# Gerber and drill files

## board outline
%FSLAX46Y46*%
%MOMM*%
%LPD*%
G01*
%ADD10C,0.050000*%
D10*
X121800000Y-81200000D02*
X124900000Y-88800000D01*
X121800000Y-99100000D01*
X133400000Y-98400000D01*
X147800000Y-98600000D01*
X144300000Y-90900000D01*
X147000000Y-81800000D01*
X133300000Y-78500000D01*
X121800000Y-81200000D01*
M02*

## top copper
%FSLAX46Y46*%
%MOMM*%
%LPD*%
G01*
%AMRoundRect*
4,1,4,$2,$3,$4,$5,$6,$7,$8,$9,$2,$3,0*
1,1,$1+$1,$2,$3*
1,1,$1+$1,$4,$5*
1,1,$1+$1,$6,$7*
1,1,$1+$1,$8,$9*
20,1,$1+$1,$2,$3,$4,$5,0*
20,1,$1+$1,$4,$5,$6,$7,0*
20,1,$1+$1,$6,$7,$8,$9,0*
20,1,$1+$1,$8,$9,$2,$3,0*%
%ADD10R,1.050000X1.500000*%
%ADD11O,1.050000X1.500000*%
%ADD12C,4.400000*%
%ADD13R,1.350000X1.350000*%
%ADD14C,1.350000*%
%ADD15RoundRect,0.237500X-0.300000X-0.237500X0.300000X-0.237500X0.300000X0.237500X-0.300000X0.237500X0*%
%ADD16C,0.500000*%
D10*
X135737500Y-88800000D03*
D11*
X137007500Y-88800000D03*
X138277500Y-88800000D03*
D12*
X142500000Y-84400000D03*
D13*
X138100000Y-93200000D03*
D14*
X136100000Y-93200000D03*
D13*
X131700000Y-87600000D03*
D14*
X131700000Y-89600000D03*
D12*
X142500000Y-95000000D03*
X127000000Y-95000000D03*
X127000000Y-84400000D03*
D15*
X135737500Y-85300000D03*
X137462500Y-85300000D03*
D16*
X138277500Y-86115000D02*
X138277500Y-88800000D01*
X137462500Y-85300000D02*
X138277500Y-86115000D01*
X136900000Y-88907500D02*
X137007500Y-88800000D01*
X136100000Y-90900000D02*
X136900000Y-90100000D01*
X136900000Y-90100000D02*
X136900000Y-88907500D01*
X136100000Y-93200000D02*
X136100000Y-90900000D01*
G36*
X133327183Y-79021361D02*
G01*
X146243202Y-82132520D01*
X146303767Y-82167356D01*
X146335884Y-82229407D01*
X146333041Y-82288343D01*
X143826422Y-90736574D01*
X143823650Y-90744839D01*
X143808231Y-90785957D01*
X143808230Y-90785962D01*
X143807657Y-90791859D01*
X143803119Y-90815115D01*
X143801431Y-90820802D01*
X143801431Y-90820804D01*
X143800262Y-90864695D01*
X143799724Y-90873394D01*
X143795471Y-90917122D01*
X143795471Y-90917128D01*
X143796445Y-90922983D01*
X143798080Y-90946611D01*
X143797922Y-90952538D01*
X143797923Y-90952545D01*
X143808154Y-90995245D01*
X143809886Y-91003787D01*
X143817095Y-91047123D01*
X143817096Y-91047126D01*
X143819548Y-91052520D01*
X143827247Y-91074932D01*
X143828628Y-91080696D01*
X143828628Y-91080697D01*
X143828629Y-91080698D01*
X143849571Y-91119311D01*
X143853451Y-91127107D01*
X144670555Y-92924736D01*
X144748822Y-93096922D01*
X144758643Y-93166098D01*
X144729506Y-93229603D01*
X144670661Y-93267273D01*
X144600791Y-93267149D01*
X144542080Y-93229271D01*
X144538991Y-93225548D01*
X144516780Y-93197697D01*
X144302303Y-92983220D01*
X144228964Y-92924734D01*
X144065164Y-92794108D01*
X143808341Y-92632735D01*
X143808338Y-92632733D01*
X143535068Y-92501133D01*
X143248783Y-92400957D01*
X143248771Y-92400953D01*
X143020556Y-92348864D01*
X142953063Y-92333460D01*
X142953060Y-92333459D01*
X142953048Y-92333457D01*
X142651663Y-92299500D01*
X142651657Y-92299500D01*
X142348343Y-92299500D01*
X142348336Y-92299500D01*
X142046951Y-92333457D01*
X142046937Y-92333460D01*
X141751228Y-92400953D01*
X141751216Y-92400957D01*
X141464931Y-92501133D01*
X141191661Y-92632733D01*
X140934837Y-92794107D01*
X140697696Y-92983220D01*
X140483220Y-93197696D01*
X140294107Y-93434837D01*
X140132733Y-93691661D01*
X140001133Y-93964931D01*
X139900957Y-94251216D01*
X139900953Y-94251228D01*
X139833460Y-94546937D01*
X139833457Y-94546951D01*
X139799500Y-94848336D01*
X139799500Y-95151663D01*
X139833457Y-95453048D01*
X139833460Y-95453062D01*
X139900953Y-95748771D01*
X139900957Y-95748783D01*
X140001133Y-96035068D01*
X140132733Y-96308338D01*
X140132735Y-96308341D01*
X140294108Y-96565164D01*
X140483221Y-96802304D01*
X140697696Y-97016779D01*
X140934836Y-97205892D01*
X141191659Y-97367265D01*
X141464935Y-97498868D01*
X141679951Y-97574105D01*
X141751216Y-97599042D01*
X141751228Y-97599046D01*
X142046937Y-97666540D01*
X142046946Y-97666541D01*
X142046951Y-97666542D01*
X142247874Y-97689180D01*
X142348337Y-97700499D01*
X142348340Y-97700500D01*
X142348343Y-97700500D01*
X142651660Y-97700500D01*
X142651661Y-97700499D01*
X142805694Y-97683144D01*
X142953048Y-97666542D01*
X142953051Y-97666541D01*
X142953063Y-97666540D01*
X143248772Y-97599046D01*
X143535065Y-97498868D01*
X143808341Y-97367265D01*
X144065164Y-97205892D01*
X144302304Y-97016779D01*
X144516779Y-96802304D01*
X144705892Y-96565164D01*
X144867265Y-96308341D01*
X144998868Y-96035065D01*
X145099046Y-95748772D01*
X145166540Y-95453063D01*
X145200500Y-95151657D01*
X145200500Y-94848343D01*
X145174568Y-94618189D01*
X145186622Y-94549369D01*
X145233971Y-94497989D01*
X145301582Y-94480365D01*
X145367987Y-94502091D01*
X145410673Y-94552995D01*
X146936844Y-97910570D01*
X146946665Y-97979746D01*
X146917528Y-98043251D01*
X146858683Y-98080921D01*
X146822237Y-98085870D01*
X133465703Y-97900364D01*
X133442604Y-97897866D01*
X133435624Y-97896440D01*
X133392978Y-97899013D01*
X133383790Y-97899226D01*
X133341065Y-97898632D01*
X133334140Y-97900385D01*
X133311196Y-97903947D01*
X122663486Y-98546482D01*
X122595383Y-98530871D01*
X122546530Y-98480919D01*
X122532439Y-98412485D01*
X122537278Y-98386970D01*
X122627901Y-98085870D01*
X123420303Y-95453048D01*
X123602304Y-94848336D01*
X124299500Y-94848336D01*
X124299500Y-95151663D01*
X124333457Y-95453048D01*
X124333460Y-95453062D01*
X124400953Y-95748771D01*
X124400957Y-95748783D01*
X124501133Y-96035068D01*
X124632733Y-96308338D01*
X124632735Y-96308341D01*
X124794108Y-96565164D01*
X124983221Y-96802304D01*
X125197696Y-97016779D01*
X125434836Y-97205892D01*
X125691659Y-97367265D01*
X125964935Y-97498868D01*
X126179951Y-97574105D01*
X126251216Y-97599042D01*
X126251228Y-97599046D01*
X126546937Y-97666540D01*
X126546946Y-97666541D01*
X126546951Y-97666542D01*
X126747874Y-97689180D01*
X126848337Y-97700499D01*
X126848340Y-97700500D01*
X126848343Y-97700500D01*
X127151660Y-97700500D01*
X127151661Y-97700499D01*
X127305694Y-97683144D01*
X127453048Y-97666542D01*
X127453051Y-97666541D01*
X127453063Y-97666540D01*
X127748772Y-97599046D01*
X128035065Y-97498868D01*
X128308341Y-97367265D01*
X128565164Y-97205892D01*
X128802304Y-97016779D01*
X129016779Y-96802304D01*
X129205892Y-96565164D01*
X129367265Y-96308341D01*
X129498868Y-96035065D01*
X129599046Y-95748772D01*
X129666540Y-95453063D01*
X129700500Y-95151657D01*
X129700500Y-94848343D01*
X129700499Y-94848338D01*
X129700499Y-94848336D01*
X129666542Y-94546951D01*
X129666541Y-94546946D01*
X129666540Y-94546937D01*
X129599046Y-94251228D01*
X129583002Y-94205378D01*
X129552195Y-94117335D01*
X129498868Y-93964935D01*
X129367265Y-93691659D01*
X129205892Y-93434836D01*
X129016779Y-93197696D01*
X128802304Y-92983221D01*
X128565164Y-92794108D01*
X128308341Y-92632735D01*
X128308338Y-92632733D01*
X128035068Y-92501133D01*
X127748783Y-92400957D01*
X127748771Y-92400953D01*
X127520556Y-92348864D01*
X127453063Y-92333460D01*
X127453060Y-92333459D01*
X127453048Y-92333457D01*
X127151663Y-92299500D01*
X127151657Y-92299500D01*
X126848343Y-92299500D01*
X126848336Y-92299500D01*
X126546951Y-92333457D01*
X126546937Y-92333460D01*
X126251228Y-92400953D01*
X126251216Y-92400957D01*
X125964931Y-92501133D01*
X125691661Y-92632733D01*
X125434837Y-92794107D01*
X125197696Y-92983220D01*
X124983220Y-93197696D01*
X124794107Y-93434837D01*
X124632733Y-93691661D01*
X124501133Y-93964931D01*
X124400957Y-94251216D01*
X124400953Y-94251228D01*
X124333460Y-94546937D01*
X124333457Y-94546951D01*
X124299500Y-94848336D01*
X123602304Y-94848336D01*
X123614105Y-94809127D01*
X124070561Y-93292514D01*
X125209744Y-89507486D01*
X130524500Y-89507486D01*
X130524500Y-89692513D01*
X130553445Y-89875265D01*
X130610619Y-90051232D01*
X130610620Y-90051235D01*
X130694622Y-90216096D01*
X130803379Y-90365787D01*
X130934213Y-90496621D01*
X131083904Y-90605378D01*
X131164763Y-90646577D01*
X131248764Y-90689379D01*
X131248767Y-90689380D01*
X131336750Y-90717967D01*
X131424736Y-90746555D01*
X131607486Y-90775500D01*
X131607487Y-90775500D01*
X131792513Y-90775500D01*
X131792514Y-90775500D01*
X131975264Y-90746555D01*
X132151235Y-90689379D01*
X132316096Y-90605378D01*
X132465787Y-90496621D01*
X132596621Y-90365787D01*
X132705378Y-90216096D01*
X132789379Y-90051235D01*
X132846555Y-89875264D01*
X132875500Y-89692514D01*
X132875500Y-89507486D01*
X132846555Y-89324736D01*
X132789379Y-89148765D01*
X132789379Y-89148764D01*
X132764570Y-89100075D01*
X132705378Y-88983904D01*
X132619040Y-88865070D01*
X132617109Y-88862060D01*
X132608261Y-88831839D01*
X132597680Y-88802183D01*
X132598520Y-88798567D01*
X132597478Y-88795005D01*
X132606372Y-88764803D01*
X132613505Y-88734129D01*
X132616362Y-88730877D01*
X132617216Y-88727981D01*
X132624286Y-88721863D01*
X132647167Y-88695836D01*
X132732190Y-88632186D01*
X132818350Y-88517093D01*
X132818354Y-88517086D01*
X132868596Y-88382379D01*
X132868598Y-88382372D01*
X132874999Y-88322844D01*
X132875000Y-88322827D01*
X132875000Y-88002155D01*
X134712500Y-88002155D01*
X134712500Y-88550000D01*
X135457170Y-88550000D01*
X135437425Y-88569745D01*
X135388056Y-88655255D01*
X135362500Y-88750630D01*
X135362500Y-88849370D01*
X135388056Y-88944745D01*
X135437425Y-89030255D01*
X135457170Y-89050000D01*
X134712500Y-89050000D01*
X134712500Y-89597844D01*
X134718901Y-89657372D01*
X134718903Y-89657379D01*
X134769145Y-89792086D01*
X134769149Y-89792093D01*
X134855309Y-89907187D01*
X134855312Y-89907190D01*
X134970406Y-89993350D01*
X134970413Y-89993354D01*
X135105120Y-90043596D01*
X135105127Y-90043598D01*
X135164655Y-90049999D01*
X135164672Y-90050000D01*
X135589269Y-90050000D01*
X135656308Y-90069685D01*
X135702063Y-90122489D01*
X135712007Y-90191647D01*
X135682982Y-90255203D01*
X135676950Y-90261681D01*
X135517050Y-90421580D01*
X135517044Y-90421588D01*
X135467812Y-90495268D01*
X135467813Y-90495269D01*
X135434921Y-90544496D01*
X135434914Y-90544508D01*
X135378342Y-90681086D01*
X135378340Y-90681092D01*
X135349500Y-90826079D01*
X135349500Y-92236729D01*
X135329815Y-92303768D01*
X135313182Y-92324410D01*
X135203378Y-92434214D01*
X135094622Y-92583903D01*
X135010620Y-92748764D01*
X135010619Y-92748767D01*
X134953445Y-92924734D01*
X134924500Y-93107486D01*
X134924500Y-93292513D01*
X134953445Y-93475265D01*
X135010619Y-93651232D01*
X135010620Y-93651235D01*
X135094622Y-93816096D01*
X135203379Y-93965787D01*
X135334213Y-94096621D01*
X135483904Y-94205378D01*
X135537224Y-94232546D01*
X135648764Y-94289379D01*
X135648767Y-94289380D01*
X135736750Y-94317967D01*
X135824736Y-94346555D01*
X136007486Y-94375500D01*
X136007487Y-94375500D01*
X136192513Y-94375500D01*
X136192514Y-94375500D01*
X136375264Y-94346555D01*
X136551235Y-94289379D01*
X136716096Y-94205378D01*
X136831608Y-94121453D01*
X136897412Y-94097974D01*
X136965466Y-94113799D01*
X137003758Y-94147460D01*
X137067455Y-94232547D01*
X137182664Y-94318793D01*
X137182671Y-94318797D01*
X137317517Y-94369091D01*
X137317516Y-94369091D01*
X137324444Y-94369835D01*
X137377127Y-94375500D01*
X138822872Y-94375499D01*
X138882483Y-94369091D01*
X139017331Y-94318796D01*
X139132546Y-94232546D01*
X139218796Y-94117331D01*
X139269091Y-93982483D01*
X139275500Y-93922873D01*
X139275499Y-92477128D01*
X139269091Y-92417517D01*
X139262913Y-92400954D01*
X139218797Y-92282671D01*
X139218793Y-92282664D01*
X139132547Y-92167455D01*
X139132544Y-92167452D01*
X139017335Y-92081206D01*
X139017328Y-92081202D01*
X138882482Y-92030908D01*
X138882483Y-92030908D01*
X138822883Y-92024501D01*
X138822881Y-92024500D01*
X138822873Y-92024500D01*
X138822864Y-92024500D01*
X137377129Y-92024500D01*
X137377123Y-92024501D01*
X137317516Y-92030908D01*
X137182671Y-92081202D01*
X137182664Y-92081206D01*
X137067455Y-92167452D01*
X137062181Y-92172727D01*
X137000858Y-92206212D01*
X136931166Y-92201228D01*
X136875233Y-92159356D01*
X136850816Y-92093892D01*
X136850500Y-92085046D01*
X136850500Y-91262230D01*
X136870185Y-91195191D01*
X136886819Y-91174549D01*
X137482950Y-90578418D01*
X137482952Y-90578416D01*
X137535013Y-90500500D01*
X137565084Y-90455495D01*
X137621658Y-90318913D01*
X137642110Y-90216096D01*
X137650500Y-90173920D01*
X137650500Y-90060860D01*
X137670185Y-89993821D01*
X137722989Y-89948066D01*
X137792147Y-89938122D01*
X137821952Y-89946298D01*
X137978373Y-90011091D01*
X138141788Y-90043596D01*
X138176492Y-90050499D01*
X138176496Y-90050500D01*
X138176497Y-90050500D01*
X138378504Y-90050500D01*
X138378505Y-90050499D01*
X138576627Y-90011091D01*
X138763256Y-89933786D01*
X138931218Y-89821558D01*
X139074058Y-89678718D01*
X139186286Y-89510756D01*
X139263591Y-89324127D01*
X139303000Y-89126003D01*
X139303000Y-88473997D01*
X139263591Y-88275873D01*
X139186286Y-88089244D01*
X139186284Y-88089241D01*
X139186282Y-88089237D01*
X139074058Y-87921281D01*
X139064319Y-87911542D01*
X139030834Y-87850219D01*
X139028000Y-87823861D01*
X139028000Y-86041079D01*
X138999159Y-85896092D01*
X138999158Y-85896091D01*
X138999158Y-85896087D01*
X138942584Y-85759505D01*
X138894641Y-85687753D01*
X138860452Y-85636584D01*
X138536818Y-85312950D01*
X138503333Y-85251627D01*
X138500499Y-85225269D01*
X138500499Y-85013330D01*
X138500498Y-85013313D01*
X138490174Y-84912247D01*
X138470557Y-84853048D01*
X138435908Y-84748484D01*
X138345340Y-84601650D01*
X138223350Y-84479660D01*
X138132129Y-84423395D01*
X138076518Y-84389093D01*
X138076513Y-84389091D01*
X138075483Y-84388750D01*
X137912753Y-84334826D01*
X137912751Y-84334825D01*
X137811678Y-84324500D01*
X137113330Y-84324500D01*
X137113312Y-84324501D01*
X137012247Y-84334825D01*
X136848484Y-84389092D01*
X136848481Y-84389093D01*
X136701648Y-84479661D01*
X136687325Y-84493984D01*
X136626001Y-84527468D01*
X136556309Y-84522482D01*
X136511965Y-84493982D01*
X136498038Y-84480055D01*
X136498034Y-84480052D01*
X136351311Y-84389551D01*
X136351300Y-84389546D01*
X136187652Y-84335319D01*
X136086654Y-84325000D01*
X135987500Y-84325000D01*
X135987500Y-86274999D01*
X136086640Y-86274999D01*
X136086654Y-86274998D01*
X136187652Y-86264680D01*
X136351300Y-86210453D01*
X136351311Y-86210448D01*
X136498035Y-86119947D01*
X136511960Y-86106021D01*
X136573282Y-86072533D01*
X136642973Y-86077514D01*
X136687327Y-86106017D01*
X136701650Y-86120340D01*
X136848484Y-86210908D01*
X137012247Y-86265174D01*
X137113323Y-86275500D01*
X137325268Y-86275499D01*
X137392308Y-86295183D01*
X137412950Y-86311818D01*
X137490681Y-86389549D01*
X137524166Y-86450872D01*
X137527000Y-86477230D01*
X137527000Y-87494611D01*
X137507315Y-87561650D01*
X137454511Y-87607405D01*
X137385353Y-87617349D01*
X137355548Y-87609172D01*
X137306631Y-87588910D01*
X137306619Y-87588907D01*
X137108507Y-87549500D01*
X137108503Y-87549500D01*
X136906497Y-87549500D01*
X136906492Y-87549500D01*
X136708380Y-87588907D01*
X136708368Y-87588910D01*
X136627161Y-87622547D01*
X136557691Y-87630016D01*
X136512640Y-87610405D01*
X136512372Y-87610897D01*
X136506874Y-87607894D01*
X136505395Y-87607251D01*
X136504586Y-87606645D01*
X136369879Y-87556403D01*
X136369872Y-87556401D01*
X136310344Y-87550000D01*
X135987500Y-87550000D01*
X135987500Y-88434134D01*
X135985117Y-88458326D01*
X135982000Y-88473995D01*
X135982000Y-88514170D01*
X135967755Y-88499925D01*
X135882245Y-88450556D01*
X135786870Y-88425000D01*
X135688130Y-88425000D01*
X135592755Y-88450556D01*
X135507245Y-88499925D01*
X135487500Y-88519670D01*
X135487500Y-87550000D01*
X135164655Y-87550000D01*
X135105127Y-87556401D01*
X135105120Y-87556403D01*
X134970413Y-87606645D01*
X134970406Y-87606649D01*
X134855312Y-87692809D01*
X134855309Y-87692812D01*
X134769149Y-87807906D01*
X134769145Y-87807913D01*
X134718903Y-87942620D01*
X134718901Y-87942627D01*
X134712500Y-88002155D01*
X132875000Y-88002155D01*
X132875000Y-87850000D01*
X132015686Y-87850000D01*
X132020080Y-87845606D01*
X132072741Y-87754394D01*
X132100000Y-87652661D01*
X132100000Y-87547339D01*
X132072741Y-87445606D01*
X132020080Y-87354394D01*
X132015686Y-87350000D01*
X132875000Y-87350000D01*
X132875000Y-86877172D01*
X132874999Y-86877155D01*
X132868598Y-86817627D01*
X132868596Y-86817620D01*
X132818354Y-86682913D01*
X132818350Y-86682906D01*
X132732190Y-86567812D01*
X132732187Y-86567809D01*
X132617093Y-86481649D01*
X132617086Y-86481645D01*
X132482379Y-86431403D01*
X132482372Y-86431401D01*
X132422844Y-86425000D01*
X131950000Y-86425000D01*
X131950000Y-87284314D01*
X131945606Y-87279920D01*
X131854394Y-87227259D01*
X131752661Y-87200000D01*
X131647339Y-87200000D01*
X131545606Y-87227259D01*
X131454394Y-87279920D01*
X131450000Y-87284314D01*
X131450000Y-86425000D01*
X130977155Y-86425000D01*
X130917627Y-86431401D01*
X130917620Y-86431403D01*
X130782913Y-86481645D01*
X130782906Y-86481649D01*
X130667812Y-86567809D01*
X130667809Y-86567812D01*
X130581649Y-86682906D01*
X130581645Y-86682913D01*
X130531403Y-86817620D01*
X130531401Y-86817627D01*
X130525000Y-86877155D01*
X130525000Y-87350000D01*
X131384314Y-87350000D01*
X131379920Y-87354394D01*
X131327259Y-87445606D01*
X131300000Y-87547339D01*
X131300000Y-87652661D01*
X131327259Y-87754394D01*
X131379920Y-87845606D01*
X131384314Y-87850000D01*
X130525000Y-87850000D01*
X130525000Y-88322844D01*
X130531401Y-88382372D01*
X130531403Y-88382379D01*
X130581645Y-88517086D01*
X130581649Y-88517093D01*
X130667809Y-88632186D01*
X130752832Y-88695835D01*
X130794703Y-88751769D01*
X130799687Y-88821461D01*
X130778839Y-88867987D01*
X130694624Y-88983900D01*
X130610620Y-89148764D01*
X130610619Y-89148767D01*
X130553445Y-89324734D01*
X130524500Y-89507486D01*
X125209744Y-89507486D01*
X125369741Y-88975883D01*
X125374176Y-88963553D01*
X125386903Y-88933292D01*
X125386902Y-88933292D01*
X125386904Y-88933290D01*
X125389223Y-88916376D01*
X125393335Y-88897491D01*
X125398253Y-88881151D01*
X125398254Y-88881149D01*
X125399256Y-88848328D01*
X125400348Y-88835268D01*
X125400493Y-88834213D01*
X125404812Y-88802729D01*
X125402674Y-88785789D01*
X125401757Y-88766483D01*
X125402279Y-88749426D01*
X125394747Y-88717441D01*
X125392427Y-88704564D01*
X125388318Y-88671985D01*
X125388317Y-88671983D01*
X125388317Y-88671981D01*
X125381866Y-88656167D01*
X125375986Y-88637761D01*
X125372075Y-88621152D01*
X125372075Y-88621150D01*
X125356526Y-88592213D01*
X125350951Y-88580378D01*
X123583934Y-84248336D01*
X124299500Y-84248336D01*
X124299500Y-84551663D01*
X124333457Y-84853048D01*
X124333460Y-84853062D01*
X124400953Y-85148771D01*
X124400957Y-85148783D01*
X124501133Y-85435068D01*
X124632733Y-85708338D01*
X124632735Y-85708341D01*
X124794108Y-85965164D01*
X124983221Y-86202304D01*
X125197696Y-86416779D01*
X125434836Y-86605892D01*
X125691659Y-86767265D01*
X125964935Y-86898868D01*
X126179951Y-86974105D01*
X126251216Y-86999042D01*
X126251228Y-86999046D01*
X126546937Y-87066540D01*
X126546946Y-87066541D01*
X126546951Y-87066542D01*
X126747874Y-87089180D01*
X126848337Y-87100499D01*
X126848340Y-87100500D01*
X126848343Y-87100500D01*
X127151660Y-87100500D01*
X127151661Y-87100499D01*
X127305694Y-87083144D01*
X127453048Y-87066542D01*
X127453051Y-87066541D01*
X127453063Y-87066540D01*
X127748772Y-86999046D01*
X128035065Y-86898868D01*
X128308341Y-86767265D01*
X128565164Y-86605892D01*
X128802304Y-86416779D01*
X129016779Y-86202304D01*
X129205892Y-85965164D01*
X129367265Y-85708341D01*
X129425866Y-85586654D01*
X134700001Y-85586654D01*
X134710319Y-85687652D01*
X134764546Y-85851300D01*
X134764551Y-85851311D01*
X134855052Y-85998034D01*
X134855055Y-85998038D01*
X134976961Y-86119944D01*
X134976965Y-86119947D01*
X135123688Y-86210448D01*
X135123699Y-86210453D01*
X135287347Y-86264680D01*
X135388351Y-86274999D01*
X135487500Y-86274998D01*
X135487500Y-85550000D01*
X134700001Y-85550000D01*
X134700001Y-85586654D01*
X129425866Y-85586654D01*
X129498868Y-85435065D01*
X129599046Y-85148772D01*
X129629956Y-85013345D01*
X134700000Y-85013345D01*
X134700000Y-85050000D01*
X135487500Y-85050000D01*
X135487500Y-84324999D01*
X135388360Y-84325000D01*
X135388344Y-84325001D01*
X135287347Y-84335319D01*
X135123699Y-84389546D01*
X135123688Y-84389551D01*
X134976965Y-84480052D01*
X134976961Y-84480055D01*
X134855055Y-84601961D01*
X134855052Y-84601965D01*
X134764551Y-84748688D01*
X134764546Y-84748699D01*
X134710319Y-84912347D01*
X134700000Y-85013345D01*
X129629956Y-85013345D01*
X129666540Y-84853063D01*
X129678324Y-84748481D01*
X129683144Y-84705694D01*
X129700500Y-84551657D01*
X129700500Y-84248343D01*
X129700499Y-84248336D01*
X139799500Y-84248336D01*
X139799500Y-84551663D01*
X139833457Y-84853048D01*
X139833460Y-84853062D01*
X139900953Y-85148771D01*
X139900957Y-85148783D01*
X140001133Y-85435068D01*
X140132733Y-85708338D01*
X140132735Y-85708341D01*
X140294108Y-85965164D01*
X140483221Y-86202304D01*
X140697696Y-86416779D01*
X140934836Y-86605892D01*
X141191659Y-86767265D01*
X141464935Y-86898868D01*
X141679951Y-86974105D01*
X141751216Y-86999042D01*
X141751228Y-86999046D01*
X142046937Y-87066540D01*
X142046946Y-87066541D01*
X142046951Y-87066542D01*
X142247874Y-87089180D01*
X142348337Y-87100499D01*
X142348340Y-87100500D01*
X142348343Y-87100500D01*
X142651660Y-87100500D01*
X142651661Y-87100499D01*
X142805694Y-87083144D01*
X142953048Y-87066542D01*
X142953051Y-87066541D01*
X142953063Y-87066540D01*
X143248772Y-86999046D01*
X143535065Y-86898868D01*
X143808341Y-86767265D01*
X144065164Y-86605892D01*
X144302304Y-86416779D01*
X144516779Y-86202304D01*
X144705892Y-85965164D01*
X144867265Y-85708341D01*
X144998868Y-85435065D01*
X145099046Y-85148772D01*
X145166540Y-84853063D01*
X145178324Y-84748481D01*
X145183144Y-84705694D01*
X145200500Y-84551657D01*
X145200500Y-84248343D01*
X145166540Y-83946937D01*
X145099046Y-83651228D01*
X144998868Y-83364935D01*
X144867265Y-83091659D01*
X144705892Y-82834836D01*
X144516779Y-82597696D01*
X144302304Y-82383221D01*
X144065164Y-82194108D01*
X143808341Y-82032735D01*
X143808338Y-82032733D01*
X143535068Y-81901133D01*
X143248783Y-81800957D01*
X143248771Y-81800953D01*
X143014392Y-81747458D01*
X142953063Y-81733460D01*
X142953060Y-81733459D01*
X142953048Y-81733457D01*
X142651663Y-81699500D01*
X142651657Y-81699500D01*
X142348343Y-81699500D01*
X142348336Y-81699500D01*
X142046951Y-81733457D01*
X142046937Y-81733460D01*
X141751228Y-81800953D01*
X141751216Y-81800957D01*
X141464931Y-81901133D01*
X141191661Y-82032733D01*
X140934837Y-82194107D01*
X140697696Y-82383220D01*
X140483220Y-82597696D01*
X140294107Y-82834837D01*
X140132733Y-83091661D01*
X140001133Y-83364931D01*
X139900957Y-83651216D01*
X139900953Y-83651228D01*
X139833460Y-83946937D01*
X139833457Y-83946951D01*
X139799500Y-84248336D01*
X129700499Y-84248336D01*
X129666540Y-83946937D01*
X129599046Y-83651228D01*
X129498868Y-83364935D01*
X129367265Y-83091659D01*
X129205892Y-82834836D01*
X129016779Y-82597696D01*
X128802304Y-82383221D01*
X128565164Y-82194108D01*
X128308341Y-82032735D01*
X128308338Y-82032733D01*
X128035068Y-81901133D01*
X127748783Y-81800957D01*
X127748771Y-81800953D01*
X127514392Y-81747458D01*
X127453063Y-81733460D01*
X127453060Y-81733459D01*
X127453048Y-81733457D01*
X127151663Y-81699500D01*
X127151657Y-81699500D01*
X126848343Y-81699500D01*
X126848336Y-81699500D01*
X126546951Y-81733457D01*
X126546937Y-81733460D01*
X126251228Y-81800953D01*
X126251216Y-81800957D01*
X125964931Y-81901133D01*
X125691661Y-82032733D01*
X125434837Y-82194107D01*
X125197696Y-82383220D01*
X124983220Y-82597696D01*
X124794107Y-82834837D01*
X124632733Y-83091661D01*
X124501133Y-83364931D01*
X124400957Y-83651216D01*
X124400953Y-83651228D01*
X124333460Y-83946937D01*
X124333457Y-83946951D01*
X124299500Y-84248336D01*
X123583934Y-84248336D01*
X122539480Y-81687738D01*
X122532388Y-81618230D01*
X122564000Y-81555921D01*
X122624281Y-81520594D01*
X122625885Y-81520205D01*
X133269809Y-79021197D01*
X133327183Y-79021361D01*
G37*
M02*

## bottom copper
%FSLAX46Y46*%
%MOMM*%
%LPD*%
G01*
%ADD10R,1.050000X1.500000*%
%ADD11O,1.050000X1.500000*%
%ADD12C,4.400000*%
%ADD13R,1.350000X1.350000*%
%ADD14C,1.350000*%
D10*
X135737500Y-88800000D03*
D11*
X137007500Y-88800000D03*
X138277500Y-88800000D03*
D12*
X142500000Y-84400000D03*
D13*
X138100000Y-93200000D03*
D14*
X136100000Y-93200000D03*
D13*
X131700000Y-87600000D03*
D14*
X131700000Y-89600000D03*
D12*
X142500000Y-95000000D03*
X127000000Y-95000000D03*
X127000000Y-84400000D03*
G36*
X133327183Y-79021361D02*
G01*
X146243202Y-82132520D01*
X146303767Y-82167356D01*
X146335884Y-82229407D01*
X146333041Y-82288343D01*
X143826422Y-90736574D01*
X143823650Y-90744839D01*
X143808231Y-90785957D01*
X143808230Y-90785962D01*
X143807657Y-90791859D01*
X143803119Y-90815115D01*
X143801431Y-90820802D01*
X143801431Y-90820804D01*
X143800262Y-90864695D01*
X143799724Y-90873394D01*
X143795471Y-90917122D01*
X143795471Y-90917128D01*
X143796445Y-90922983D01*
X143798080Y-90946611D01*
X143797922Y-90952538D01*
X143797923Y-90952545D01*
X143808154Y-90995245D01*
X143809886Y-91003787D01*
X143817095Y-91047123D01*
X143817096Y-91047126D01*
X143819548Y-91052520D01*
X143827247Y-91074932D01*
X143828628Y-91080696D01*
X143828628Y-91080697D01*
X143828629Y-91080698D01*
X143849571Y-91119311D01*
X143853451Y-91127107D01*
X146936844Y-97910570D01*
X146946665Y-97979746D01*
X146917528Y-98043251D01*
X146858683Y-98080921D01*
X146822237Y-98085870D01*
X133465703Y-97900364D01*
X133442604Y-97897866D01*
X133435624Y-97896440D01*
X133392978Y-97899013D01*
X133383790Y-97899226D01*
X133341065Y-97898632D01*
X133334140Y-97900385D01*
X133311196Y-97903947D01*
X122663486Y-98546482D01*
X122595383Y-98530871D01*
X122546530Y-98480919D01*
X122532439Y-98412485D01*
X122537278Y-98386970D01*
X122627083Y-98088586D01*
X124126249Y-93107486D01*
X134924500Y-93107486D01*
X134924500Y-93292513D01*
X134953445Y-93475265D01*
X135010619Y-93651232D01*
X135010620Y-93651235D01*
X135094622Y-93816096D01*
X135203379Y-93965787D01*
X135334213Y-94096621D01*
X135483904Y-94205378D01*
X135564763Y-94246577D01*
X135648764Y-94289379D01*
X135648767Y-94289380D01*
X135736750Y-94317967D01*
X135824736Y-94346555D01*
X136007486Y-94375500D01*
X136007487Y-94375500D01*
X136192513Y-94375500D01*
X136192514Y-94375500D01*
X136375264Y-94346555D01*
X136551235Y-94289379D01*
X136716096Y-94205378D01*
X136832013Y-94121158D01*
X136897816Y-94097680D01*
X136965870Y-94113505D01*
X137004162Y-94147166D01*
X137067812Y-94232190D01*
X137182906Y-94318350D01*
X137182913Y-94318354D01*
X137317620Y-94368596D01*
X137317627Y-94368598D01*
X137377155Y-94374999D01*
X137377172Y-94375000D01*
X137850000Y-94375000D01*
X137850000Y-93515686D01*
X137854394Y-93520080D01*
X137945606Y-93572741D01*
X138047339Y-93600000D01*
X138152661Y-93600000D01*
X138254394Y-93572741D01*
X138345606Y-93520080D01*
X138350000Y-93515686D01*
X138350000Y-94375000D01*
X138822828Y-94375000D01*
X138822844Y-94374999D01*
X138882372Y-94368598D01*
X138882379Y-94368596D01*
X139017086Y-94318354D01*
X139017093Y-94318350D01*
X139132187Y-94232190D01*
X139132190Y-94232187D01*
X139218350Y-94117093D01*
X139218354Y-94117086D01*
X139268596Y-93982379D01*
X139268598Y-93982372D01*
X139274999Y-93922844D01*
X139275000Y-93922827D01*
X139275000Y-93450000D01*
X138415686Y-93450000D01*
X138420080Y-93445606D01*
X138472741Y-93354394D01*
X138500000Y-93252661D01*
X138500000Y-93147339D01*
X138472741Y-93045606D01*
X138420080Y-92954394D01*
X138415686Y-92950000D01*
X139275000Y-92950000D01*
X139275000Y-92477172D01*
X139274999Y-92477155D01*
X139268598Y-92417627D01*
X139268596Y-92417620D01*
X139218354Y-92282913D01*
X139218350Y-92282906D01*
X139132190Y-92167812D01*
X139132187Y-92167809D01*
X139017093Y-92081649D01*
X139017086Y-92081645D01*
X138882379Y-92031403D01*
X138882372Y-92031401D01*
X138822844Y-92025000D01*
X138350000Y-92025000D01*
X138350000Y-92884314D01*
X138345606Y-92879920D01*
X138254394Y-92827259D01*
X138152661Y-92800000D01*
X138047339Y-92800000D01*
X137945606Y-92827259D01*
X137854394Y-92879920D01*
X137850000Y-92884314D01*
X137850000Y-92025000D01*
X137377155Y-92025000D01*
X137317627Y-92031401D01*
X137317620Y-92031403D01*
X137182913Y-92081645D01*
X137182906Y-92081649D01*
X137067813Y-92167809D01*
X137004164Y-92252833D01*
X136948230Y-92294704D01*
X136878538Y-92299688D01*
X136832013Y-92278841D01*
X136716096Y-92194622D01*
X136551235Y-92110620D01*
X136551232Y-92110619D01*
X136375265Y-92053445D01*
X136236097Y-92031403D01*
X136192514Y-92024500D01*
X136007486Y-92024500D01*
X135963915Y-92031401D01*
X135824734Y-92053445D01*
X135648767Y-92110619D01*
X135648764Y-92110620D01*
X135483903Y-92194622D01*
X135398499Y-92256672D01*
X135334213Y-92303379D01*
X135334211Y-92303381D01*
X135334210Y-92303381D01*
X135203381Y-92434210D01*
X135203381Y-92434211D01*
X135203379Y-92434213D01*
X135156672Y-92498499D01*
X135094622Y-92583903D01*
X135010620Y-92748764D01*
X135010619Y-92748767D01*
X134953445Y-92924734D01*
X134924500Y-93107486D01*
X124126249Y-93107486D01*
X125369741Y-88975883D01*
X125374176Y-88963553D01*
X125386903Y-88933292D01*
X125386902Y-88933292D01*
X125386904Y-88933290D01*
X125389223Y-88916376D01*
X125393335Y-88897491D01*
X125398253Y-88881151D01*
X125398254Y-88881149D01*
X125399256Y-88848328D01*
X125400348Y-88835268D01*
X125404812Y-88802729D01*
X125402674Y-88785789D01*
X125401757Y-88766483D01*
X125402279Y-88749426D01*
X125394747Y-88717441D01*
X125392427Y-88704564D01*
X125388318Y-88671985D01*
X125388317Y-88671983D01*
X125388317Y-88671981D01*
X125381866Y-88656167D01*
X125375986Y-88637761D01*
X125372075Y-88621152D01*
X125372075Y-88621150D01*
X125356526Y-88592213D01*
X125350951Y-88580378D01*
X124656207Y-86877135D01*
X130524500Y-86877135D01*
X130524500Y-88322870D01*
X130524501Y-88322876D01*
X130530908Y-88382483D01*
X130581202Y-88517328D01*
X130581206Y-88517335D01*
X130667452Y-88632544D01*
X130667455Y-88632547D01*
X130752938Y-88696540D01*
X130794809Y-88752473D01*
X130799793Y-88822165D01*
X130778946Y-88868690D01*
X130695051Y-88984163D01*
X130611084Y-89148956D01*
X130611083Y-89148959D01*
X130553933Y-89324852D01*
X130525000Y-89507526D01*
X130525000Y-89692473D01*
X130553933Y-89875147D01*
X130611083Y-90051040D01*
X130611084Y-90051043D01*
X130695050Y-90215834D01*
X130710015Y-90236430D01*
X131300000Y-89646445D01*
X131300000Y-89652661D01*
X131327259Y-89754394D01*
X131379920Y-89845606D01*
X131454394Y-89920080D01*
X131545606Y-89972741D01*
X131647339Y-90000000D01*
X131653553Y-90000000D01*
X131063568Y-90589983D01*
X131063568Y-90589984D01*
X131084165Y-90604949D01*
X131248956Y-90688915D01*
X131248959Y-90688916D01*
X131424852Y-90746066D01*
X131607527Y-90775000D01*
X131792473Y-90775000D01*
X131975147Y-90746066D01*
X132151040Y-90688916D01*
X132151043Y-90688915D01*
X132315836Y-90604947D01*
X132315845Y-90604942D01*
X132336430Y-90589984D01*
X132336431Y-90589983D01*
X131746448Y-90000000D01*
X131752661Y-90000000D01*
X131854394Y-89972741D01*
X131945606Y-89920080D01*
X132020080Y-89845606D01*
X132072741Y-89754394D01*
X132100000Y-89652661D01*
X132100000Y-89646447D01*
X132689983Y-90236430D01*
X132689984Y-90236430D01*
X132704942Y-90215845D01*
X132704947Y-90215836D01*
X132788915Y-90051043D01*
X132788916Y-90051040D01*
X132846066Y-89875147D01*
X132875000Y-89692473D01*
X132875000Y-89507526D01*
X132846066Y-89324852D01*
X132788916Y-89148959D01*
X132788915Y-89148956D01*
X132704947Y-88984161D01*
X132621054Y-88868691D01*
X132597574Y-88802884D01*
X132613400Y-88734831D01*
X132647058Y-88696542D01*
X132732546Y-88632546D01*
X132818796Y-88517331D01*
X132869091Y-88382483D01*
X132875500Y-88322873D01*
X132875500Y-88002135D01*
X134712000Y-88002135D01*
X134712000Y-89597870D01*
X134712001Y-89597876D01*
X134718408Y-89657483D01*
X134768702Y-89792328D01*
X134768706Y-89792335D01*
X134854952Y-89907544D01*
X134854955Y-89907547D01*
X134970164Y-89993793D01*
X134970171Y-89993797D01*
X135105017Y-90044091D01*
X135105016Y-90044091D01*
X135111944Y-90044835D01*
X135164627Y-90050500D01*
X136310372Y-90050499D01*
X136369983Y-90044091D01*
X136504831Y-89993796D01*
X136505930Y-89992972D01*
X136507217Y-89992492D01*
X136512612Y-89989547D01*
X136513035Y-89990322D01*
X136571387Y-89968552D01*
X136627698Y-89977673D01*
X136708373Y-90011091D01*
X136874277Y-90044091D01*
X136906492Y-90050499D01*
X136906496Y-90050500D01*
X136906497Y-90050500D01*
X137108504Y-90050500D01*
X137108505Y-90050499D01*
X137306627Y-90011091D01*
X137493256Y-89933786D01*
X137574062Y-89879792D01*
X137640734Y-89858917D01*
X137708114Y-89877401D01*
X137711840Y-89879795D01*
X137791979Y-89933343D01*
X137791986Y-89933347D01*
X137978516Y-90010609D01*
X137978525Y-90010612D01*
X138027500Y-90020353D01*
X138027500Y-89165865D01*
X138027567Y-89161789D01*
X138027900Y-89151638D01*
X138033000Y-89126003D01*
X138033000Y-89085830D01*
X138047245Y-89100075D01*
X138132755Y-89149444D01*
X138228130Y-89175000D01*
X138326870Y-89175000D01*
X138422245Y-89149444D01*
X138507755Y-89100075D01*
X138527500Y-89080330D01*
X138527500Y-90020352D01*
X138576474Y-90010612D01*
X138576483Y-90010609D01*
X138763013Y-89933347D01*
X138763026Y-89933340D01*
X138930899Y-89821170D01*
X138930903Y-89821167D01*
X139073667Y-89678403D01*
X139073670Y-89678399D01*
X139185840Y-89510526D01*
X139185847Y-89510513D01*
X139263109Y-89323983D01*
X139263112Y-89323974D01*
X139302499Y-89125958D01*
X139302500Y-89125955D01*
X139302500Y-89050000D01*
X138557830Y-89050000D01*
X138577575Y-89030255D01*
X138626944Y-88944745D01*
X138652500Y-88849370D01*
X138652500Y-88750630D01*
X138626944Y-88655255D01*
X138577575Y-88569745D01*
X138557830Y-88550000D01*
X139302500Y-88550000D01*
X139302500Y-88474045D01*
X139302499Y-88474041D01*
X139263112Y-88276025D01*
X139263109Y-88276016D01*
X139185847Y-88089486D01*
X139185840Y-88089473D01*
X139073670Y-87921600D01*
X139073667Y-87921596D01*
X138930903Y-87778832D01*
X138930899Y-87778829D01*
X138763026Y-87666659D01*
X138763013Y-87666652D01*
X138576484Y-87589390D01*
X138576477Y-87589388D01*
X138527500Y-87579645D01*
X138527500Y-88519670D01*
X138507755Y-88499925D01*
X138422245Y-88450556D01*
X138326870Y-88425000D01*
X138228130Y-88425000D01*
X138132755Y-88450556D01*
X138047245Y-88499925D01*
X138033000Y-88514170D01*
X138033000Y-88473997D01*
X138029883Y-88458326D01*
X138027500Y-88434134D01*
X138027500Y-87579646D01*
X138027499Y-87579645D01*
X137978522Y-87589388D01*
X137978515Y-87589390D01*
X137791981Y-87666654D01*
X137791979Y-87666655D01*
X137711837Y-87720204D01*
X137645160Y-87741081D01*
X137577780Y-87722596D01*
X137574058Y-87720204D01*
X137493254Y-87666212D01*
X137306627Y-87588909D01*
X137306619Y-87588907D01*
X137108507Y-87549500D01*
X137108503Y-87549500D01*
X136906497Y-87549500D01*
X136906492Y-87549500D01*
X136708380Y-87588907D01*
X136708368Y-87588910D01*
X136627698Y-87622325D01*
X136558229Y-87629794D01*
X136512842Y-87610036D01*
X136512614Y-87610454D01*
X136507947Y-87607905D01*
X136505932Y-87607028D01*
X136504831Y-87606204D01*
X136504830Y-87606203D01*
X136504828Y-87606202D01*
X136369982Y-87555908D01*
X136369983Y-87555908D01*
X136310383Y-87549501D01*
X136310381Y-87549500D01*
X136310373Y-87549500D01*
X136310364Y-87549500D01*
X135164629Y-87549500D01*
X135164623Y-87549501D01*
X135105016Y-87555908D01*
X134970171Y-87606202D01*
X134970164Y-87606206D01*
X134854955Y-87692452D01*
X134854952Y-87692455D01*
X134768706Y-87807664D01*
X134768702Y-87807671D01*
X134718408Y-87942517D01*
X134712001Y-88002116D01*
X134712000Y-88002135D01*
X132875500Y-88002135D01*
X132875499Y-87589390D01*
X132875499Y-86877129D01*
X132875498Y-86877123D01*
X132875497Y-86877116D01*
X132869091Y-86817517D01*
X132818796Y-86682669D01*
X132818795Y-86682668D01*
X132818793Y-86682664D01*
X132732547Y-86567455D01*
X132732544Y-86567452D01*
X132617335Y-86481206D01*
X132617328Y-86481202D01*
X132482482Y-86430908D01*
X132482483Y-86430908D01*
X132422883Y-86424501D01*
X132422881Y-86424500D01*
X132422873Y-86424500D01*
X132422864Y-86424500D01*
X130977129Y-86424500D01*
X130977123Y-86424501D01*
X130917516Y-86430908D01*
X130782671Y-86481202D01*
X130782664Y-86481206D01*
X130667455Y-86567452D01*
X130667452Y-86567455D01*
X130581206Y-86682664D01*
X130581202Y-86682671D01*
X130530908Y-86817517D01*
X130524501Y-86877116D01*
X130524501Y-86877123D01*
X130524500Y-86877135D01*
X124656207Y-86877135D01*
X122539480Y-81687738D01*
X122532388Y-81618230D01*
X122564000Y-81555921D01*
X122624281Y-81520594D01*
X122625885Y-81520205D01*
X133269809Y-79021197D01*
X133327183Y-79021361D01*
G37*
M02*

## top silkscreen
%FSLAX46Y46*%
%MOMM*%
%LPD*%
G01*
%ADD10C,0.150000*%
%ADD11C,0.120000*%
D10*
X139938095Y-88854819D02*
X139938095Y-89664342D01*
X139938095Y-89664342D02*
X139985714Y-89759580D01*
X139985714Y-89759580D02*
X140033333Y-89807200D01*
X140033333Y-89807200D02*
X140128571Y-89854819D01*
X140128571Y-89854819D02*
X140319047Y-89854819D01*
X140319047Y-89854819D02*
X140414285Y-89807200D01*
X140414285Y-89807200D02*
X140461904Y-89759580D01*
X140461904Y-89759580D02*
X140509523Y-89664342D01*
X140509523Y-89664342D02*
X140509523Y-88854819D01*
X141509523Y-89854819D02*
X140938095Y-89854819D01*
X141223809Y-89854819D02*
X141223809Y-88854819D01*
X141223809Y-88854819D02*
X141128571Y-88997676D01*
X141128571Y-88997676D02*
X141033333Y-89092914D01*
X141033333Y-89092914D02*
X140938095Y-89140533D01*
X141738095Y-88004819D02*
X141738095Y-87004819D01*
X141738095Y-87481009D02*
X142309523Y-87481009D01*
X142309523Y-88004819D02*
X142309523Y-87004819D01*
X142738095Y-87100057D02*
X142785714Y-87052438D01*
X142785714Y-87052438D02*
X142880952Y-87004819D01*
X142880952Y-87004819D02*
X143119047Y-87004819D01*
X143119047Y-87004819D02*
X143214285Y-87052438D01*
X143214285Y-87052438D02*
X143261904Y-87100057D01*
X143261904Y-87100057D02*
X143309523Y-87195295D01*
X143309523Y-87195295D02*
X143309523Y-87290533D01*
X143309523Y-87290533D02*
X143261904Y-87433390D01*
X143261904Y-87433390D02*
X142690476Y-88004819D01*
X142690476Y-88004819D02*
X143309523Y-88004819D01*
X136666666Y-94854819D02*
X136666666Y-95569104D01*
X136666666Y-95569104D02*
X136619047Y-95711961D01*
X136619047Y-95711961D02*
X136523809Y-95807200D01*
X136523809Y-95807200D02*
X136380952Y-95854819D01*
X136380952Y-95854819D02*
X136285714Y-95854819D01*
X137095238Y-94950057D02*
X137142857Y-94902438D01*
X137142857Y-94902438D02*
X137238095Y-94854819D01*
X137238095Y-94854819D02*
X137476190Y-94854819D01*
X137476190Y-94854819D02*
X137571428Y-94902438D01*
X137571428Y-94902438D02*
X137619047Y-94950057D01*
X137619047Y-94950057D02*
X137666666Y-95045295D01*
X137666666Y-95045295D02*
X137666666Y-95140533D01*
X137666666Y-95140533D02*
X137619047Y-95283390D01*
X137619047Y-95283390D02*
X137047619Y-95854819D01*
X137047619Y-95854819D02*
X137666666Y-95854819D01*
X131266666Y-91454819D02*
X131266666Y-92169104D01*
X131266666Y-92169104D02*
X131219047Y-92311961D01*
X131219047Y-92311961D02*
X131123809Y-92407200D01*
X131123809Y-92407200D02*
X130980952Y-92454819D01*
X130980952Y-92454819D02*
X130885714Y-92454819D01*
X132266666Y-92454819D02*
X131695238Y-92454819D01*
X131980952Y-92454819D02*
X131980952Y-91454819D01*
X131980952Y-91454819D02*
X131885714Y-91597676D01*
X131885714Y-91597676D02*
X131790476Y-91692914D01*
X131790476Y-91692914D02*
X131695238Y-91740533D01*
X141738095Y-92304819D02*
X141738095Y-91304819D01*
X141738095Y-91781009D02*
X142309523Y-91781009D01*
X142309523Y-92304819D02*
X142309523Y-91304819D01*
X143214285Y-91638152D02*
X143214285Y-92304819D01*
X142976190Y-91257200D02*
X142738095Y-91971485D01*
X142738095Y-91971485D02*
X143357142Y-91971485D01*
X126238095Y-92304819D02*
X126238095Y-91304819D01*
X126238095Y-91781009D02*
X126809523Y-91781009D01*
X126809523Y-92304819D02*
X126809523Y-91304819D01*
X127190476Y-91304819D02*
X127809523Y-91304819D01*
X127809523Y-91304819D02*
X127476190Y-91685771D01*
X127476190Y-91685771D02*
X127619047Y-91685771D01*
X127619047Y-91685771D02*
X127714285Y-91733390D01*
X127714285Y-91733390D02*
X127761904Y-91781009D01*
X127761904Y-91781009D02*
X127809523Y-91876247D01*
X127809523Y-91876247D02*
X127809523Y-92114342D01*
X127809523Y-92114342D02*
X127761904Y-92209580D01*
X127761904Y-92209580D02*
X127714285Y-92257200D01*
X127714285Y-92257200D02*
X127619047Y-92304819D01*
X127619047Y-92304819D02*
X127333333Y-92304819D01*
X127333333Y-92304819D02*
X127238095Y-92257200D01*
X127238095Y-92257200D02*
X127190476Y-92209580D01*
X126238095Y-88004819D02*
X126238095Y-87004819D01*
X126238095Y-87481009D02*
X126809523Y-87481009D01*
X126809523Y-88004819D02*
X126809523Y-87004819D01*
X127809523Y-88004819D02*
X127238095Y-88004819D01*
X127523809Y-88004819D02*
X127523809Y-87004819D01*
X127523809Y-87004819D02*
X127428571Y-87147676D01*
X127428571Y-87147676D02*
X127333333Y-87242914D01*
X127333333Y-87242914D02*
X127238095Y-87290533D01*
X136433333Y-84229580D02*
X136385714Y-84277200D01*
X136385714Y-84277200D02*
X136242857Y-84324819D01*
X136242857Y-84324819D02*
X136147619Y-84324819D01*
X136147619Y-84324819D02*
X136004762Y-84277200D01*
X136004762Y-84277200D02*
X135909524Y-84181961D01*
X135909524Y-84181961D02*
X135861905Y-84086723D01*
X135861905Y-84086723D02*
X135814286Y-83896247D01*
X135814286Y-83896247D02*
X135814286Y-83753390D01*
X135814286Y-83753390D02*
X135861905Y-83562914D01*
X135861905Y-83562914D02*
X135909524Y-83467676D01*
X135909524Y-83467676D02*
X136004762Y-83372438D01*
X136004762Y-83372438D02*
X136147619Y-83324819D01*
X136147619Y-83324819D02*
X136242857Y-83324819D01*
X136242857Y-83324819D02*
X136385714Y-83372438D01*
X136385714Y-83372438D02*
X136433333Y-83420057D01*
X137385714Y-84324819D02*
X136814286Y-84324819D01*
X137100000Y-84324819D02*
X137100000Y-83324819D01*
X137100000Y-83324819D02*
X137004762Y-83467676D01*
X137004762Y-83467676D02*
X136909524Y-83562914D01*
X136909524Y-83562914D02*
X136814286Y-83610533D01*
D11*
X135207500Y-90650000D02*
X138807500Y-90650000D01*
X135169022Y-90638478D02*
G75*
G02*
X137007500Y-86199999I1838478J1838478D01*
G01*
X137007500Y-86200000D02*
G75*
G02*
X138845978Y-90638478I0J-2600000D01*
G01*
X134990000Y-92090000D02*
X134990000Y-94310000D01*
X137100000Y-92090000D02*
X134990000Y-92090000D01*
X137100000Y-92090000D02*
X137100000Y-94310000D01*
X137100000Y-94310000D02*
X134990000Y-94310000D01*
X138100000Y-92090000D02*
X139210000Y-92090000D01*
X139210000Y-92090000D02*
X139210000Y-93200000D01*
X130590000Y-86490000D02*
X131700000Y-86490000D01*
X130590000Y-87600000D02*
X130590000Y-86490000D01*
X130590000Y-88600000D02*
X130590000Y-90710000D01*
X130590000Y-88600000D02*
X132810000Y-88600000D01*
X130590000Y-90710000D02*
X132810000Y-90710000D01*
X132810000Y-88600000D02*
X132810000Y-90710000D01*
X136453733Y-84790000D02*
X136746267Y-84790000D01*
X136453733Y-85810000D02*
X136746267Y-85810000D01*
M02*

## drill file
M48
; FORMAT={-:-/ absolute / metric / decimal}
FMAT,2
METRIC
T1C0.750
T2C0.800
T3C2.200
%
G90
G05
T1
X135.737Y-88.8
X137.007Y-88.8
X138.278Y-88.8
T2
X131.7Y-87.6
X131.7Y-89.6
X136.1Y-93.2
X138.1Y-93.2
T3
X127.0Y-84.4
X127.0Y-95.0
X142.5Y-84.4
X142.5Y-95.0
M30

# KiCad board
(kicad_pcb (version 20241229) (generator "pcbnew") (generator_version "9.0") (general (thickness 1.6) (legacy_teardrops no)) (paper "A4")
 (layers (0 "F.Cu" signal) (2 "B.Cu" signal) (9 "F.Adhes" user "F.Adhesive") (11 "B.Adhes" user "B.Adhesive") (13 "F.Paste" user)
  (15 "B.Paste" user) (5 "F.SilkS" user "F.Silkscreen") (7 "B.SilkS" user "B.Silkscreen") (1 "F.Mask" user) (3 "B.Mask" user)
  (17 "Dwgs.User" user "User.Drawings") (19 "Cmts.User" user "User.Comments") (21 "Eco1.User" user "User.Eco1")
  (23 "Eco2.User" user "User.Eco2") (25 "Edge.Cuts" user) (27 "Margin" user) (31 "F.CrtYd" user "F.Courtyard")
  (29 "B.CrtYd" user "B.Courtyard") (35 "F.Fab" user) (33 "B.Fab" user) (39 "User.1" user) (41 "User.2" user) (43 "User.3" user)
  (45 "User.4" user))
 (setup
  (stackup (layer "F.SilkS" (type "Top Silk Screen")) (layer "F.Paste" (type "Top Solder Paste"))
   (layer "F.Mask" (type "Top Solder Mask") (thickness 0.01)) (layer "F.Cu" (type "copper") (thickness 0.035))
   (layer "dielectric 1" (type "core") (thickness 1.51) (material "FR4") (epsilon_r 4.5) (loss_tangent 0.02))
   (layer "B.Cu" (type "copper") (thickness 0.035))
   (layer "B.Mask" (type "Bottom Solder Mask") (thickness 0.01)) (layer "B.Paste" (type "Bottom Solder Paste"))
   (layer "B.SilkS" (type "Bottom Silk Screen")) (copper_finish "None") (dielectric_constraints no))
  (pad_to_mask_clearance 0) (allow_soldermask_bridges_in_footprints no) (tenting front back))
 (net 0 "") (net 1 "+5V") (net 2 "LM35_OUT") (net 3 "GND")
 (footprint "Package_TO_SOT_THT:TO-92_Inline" (layer "F.Cu") (at 135.7375 88.8)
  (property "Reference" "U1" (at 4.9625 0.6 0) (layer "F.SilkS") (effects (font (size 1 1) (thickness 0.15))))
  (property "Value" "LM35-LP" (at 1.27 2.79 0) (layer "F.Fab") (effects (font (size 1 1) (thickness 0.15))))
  (fp_line (start -0.53 1.85) (end 3.07 1.85) (stroke (width 0.12) (type solid)) (layer "F.SilkS"))
  (fp_arc (start -0.568478 1.838478) (mid -1.132087 -0.994977) (end 1.27 -2.6) (stroke (width 0.12) (type solid)) (layer "F.SilkS"))
  (fp_arc (start 1.27 -2.6) (mid 3.672087 -0.994977) (end 3.108478 1.838478) (stroke (width 0.12) (type solid)) (layer "F.SilkS"))
  (pad "1" thru_hole rect (at 0 0) (size 1.05 1.5) (drill 0.75) (layers "*.Cu" "*.Mask") (remove_unused_layers no) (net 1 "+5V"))
  (pad "2" thru_hole oval (at 1.27 0) (size 1.05 1.5) (drill 0.75) (layers "*.Cu" "*.Mask") (remove_unused_layers no) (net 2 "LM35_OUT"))
  (pad "3" thru_hole oval (at 2.54 0) (size 1.05 1.5) (drill 0.75) (layers "*.Cu" "*.Mask") (remove_unused_layers no) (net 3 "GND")))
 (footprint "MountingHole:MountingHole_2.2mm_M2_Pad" (layer "F.Cu") (at 142.5 84.4 180)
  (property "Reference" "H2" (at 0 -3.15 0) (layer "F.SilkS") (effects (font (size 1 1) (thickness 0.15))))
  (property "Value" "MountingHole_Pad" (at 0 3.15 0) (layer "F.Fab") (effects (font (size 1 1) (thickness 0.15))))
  (pad "1" thru_hole circle (at 0 0 180) (size 4.4 4.4) (drill 2.2) (layers "*.Cu" "*.Mask") (remove_unused_layers no) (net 3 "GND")
   (zone_connect 2)))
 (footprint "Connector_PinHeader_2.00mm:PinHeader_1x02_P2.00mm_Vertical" (layer "F.Cu") (at 138.1 93.2 -90)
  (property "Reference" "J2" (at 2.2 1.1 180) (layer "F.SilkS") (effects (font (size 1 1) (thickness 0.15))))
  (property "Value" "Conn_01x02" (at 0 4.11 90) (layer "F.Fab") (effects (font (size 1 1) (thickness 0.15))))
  (fp_line (start -1.11 3.11) (end 1.11 3.11) (stroke (width 0.12) (type solid)) (layer "F.SilkS"))
  (fp_line (start -1.11 1) (end -1.11 3.11) (stroke (width 0.12) (type solid)) (layer "F.SilkS"))
  (fp_line (start -1.11 1) (end 1.11 1) (stroke (width 0.12) (type solid)) (layer "F.SilkS"))
  (fp_line (start 1.11 1) (end 1.11 3.11) (stroke (width 0.12) (type solid)) (layer "F.SilkS"))
  (fp_line (start -1.11 0) (end -1.11 -1.11) (stroke (width 0.12) (type solid)) (layer "F.SilkS"))
  (fp_line (start -1.11 -1.11) (end 0 -1.11) (stroke (width 0.12) (type solid)) (layer "F.SilkS"))
  (pad "1" thru_hole rect (at 0 0 270) (size 1.35 1.35) (drill 0.8) (layers "*.Cu" "*.Mask") (remove_unused_layers no) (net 3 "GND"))
  (pad "2" thru_hole circle (at 0 2 270) (size 1.35 1.35) (drill 0.8) (layers "*.Cu" "*.Mask") (remove_unused_layers no) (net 2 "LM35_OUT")))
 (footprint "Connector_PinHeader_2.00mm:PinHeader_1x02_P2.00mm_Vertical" (layer "F.Cu") (at 131.7 87.6)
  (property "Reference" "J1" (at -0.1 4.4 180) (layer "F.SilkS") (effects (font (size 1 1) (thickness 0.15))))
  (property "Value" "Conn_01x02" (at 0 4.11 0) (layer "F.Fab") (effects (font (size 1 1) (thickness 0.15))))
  (fp_line (start -1.11 -1.11) (end 0 -1.11) (stroke (width 0.12) (type solid)) (layer "F.SilkS"))
  (fp_line (start -1.11 0) (end -1.11 -1.11) (stroke (width 0.12) (type solid)) (layer "F.SilkS"))
  (fp_line (start -1.11 1) (end -1.11 3.11) (stroke (width 0.12) (type solid)) (layer "F.SilkS"))
  (fp_line (start -1.11 1) (end 1.11 1) (stroke (width 0.12) (type solid)) (layer "F.SilkS"))
  (fp_line (start -1.11 3.11) (end 1.11 3.11) (stroke (width 0.12) (type solid)) (layer "F.SilkS"))
  (fp_line (start 1.11 1) (end 1.11 3.11) (stroke (width 0.12) (type solid)) (layer "F.SilkS"))
  (pad "1" thru_hole rect (at 0 0) (size 1.35 1.35) (drill 0.8) (layers "*.Cu" "*.Mask") (remove_unused_layers no) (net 1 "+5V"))
  (pad "2" thru_hole circle (at 0 2) (size 1.35 1.35) (drill 0.8) (layers "*.Cu" "*.Mask") (remove_unused_layers no) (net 3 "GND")))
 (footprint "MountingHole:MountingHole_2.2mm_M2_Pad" (layer "F.Cu") (at 142.5 95)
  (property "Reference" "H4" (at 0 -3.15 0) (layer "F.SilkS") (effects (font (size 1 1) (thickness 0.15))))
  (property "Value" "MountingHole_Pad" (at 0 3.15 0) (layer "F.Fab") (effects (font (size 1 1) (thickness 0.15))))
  (pad "1" thru_hole circle (at 0 0) (size 4.4 4.4) (drill 2.2) (layers "*.Cu" "*.Mask") (remove_unused_layers no) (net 3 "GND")
   (zone_connect 2)))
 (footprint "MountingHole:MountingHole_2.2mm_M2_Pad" (layer "F.Cu") (at 127 95)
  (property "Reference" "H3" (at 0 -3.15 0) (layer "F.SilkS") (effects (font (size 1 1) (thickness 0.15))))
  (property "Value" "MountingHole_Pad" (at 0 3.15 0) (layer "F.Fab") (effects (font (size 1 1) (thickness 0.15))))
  (pad "1" thru_hole circle (at 0 0) (size 4.4 4.4) (drill 2.2) (layers "*.Cu" "*.Mask") (remove_unused_layers no) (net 3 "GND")
   (zone_connect 2)))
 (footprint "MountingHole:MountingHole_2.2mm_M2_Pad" (layer "F.Cu") (at 127 84.4 180)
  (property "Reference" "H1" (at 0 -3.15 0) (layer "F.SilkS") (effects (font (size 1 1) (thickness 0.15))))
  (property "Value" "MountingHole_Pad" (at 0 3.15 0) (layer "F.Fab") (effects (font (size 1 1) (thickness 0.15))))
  (pad "1" thru_hole circle (at 0 0 180) (size 4.4 4.4) (drill 2.2) (layers "*.Cu" "*.Mask") (remove_unused_layers no) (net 3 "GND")
   (zone_connect 2)))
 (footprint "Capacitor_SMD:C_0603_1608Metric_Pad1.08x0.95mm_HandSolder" (layer "F.Cu") (at 136.6 85.3)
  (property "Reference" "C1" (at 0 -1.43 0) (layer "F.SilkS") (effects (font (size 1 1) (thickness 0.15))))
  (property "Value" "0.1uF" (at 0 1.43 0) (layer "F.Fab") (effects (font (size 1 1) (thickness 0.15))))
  (fp_line (start -0.146267 -0.51) (end 0.146267 -0.51) (stroke (width 0.12) (type solid)) (layer "F.SilkS"))
  (fp_line (start -0.146267 0.51) (end 0.146267 0.51) (stroke (width 0.12) (type solid)) (layer "F.SilkS"))
  (pad "1" smd roundrect (at -0.8625 0) (size 1.075 0.95) (layers "F.Cu" "F.Mask" "F.Paste") (roundrect_rratio 0.25) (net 1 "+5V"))
  (pad "2" smd roundrect (at 0.8625 0) (size 1.075 0.95) (layers "F.Cu" "F.Mask" "F.Paste") (roundrect_rratio 0.25) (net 3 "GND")))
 (gr_poly
  (pts (xy 121.8 81.2) (xy 124.9 88.8) (xy 121.8 99.1) (xy 133.4 98.4) (xy 147.8 98.6) (xy 144.3 90.9) (xy 147 81.8) (xy 133.3 78.5))
  (stroke (width 0.05) (type solid)) (fill no) (layer "Edge.Cuts"))
 (segment (start 138.2775 86.115) (end 138.2775 88.8) (width 0.5) (layer "F.Cu") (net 3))
 (segment (start 137.4625 85.3) (end 138.2775 86.115) (width 0.5) (layer "F.Cu") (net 3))
 (segment (start 136.9 88.9075) (end 137.0075 88.8) (width 0.5) (layer "F.Cu") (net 2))
 (segment (start 136.1 90.9) (end 136.9 90.1) (width 0.5) (layer "F.Cu") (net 2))
 (segment (start 136.9 90.1) (end 136.9 88.9075) (width 0.5) (layer "F.Cu") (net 2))
 (segment (start 136.1 93.2) (end 136.1 90.9) (width 0.5) (layer "F.Cu") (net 2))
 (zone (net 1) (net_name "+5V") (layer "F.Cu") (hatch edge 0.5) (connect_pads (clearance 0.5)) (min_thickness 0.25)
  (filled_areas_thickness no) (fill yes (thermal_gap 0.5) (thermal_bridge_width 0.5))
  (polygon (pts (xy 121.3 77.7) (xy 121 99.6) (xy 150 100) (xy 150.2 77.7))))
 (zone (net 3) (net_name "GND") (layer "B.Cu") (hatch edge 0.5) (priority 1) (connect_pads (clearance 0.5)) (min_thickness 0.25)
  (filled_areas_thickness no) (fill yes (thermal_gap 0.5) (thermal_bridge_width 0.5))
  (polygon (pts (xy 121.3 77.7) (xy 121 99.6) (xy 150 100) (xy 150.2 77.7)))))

